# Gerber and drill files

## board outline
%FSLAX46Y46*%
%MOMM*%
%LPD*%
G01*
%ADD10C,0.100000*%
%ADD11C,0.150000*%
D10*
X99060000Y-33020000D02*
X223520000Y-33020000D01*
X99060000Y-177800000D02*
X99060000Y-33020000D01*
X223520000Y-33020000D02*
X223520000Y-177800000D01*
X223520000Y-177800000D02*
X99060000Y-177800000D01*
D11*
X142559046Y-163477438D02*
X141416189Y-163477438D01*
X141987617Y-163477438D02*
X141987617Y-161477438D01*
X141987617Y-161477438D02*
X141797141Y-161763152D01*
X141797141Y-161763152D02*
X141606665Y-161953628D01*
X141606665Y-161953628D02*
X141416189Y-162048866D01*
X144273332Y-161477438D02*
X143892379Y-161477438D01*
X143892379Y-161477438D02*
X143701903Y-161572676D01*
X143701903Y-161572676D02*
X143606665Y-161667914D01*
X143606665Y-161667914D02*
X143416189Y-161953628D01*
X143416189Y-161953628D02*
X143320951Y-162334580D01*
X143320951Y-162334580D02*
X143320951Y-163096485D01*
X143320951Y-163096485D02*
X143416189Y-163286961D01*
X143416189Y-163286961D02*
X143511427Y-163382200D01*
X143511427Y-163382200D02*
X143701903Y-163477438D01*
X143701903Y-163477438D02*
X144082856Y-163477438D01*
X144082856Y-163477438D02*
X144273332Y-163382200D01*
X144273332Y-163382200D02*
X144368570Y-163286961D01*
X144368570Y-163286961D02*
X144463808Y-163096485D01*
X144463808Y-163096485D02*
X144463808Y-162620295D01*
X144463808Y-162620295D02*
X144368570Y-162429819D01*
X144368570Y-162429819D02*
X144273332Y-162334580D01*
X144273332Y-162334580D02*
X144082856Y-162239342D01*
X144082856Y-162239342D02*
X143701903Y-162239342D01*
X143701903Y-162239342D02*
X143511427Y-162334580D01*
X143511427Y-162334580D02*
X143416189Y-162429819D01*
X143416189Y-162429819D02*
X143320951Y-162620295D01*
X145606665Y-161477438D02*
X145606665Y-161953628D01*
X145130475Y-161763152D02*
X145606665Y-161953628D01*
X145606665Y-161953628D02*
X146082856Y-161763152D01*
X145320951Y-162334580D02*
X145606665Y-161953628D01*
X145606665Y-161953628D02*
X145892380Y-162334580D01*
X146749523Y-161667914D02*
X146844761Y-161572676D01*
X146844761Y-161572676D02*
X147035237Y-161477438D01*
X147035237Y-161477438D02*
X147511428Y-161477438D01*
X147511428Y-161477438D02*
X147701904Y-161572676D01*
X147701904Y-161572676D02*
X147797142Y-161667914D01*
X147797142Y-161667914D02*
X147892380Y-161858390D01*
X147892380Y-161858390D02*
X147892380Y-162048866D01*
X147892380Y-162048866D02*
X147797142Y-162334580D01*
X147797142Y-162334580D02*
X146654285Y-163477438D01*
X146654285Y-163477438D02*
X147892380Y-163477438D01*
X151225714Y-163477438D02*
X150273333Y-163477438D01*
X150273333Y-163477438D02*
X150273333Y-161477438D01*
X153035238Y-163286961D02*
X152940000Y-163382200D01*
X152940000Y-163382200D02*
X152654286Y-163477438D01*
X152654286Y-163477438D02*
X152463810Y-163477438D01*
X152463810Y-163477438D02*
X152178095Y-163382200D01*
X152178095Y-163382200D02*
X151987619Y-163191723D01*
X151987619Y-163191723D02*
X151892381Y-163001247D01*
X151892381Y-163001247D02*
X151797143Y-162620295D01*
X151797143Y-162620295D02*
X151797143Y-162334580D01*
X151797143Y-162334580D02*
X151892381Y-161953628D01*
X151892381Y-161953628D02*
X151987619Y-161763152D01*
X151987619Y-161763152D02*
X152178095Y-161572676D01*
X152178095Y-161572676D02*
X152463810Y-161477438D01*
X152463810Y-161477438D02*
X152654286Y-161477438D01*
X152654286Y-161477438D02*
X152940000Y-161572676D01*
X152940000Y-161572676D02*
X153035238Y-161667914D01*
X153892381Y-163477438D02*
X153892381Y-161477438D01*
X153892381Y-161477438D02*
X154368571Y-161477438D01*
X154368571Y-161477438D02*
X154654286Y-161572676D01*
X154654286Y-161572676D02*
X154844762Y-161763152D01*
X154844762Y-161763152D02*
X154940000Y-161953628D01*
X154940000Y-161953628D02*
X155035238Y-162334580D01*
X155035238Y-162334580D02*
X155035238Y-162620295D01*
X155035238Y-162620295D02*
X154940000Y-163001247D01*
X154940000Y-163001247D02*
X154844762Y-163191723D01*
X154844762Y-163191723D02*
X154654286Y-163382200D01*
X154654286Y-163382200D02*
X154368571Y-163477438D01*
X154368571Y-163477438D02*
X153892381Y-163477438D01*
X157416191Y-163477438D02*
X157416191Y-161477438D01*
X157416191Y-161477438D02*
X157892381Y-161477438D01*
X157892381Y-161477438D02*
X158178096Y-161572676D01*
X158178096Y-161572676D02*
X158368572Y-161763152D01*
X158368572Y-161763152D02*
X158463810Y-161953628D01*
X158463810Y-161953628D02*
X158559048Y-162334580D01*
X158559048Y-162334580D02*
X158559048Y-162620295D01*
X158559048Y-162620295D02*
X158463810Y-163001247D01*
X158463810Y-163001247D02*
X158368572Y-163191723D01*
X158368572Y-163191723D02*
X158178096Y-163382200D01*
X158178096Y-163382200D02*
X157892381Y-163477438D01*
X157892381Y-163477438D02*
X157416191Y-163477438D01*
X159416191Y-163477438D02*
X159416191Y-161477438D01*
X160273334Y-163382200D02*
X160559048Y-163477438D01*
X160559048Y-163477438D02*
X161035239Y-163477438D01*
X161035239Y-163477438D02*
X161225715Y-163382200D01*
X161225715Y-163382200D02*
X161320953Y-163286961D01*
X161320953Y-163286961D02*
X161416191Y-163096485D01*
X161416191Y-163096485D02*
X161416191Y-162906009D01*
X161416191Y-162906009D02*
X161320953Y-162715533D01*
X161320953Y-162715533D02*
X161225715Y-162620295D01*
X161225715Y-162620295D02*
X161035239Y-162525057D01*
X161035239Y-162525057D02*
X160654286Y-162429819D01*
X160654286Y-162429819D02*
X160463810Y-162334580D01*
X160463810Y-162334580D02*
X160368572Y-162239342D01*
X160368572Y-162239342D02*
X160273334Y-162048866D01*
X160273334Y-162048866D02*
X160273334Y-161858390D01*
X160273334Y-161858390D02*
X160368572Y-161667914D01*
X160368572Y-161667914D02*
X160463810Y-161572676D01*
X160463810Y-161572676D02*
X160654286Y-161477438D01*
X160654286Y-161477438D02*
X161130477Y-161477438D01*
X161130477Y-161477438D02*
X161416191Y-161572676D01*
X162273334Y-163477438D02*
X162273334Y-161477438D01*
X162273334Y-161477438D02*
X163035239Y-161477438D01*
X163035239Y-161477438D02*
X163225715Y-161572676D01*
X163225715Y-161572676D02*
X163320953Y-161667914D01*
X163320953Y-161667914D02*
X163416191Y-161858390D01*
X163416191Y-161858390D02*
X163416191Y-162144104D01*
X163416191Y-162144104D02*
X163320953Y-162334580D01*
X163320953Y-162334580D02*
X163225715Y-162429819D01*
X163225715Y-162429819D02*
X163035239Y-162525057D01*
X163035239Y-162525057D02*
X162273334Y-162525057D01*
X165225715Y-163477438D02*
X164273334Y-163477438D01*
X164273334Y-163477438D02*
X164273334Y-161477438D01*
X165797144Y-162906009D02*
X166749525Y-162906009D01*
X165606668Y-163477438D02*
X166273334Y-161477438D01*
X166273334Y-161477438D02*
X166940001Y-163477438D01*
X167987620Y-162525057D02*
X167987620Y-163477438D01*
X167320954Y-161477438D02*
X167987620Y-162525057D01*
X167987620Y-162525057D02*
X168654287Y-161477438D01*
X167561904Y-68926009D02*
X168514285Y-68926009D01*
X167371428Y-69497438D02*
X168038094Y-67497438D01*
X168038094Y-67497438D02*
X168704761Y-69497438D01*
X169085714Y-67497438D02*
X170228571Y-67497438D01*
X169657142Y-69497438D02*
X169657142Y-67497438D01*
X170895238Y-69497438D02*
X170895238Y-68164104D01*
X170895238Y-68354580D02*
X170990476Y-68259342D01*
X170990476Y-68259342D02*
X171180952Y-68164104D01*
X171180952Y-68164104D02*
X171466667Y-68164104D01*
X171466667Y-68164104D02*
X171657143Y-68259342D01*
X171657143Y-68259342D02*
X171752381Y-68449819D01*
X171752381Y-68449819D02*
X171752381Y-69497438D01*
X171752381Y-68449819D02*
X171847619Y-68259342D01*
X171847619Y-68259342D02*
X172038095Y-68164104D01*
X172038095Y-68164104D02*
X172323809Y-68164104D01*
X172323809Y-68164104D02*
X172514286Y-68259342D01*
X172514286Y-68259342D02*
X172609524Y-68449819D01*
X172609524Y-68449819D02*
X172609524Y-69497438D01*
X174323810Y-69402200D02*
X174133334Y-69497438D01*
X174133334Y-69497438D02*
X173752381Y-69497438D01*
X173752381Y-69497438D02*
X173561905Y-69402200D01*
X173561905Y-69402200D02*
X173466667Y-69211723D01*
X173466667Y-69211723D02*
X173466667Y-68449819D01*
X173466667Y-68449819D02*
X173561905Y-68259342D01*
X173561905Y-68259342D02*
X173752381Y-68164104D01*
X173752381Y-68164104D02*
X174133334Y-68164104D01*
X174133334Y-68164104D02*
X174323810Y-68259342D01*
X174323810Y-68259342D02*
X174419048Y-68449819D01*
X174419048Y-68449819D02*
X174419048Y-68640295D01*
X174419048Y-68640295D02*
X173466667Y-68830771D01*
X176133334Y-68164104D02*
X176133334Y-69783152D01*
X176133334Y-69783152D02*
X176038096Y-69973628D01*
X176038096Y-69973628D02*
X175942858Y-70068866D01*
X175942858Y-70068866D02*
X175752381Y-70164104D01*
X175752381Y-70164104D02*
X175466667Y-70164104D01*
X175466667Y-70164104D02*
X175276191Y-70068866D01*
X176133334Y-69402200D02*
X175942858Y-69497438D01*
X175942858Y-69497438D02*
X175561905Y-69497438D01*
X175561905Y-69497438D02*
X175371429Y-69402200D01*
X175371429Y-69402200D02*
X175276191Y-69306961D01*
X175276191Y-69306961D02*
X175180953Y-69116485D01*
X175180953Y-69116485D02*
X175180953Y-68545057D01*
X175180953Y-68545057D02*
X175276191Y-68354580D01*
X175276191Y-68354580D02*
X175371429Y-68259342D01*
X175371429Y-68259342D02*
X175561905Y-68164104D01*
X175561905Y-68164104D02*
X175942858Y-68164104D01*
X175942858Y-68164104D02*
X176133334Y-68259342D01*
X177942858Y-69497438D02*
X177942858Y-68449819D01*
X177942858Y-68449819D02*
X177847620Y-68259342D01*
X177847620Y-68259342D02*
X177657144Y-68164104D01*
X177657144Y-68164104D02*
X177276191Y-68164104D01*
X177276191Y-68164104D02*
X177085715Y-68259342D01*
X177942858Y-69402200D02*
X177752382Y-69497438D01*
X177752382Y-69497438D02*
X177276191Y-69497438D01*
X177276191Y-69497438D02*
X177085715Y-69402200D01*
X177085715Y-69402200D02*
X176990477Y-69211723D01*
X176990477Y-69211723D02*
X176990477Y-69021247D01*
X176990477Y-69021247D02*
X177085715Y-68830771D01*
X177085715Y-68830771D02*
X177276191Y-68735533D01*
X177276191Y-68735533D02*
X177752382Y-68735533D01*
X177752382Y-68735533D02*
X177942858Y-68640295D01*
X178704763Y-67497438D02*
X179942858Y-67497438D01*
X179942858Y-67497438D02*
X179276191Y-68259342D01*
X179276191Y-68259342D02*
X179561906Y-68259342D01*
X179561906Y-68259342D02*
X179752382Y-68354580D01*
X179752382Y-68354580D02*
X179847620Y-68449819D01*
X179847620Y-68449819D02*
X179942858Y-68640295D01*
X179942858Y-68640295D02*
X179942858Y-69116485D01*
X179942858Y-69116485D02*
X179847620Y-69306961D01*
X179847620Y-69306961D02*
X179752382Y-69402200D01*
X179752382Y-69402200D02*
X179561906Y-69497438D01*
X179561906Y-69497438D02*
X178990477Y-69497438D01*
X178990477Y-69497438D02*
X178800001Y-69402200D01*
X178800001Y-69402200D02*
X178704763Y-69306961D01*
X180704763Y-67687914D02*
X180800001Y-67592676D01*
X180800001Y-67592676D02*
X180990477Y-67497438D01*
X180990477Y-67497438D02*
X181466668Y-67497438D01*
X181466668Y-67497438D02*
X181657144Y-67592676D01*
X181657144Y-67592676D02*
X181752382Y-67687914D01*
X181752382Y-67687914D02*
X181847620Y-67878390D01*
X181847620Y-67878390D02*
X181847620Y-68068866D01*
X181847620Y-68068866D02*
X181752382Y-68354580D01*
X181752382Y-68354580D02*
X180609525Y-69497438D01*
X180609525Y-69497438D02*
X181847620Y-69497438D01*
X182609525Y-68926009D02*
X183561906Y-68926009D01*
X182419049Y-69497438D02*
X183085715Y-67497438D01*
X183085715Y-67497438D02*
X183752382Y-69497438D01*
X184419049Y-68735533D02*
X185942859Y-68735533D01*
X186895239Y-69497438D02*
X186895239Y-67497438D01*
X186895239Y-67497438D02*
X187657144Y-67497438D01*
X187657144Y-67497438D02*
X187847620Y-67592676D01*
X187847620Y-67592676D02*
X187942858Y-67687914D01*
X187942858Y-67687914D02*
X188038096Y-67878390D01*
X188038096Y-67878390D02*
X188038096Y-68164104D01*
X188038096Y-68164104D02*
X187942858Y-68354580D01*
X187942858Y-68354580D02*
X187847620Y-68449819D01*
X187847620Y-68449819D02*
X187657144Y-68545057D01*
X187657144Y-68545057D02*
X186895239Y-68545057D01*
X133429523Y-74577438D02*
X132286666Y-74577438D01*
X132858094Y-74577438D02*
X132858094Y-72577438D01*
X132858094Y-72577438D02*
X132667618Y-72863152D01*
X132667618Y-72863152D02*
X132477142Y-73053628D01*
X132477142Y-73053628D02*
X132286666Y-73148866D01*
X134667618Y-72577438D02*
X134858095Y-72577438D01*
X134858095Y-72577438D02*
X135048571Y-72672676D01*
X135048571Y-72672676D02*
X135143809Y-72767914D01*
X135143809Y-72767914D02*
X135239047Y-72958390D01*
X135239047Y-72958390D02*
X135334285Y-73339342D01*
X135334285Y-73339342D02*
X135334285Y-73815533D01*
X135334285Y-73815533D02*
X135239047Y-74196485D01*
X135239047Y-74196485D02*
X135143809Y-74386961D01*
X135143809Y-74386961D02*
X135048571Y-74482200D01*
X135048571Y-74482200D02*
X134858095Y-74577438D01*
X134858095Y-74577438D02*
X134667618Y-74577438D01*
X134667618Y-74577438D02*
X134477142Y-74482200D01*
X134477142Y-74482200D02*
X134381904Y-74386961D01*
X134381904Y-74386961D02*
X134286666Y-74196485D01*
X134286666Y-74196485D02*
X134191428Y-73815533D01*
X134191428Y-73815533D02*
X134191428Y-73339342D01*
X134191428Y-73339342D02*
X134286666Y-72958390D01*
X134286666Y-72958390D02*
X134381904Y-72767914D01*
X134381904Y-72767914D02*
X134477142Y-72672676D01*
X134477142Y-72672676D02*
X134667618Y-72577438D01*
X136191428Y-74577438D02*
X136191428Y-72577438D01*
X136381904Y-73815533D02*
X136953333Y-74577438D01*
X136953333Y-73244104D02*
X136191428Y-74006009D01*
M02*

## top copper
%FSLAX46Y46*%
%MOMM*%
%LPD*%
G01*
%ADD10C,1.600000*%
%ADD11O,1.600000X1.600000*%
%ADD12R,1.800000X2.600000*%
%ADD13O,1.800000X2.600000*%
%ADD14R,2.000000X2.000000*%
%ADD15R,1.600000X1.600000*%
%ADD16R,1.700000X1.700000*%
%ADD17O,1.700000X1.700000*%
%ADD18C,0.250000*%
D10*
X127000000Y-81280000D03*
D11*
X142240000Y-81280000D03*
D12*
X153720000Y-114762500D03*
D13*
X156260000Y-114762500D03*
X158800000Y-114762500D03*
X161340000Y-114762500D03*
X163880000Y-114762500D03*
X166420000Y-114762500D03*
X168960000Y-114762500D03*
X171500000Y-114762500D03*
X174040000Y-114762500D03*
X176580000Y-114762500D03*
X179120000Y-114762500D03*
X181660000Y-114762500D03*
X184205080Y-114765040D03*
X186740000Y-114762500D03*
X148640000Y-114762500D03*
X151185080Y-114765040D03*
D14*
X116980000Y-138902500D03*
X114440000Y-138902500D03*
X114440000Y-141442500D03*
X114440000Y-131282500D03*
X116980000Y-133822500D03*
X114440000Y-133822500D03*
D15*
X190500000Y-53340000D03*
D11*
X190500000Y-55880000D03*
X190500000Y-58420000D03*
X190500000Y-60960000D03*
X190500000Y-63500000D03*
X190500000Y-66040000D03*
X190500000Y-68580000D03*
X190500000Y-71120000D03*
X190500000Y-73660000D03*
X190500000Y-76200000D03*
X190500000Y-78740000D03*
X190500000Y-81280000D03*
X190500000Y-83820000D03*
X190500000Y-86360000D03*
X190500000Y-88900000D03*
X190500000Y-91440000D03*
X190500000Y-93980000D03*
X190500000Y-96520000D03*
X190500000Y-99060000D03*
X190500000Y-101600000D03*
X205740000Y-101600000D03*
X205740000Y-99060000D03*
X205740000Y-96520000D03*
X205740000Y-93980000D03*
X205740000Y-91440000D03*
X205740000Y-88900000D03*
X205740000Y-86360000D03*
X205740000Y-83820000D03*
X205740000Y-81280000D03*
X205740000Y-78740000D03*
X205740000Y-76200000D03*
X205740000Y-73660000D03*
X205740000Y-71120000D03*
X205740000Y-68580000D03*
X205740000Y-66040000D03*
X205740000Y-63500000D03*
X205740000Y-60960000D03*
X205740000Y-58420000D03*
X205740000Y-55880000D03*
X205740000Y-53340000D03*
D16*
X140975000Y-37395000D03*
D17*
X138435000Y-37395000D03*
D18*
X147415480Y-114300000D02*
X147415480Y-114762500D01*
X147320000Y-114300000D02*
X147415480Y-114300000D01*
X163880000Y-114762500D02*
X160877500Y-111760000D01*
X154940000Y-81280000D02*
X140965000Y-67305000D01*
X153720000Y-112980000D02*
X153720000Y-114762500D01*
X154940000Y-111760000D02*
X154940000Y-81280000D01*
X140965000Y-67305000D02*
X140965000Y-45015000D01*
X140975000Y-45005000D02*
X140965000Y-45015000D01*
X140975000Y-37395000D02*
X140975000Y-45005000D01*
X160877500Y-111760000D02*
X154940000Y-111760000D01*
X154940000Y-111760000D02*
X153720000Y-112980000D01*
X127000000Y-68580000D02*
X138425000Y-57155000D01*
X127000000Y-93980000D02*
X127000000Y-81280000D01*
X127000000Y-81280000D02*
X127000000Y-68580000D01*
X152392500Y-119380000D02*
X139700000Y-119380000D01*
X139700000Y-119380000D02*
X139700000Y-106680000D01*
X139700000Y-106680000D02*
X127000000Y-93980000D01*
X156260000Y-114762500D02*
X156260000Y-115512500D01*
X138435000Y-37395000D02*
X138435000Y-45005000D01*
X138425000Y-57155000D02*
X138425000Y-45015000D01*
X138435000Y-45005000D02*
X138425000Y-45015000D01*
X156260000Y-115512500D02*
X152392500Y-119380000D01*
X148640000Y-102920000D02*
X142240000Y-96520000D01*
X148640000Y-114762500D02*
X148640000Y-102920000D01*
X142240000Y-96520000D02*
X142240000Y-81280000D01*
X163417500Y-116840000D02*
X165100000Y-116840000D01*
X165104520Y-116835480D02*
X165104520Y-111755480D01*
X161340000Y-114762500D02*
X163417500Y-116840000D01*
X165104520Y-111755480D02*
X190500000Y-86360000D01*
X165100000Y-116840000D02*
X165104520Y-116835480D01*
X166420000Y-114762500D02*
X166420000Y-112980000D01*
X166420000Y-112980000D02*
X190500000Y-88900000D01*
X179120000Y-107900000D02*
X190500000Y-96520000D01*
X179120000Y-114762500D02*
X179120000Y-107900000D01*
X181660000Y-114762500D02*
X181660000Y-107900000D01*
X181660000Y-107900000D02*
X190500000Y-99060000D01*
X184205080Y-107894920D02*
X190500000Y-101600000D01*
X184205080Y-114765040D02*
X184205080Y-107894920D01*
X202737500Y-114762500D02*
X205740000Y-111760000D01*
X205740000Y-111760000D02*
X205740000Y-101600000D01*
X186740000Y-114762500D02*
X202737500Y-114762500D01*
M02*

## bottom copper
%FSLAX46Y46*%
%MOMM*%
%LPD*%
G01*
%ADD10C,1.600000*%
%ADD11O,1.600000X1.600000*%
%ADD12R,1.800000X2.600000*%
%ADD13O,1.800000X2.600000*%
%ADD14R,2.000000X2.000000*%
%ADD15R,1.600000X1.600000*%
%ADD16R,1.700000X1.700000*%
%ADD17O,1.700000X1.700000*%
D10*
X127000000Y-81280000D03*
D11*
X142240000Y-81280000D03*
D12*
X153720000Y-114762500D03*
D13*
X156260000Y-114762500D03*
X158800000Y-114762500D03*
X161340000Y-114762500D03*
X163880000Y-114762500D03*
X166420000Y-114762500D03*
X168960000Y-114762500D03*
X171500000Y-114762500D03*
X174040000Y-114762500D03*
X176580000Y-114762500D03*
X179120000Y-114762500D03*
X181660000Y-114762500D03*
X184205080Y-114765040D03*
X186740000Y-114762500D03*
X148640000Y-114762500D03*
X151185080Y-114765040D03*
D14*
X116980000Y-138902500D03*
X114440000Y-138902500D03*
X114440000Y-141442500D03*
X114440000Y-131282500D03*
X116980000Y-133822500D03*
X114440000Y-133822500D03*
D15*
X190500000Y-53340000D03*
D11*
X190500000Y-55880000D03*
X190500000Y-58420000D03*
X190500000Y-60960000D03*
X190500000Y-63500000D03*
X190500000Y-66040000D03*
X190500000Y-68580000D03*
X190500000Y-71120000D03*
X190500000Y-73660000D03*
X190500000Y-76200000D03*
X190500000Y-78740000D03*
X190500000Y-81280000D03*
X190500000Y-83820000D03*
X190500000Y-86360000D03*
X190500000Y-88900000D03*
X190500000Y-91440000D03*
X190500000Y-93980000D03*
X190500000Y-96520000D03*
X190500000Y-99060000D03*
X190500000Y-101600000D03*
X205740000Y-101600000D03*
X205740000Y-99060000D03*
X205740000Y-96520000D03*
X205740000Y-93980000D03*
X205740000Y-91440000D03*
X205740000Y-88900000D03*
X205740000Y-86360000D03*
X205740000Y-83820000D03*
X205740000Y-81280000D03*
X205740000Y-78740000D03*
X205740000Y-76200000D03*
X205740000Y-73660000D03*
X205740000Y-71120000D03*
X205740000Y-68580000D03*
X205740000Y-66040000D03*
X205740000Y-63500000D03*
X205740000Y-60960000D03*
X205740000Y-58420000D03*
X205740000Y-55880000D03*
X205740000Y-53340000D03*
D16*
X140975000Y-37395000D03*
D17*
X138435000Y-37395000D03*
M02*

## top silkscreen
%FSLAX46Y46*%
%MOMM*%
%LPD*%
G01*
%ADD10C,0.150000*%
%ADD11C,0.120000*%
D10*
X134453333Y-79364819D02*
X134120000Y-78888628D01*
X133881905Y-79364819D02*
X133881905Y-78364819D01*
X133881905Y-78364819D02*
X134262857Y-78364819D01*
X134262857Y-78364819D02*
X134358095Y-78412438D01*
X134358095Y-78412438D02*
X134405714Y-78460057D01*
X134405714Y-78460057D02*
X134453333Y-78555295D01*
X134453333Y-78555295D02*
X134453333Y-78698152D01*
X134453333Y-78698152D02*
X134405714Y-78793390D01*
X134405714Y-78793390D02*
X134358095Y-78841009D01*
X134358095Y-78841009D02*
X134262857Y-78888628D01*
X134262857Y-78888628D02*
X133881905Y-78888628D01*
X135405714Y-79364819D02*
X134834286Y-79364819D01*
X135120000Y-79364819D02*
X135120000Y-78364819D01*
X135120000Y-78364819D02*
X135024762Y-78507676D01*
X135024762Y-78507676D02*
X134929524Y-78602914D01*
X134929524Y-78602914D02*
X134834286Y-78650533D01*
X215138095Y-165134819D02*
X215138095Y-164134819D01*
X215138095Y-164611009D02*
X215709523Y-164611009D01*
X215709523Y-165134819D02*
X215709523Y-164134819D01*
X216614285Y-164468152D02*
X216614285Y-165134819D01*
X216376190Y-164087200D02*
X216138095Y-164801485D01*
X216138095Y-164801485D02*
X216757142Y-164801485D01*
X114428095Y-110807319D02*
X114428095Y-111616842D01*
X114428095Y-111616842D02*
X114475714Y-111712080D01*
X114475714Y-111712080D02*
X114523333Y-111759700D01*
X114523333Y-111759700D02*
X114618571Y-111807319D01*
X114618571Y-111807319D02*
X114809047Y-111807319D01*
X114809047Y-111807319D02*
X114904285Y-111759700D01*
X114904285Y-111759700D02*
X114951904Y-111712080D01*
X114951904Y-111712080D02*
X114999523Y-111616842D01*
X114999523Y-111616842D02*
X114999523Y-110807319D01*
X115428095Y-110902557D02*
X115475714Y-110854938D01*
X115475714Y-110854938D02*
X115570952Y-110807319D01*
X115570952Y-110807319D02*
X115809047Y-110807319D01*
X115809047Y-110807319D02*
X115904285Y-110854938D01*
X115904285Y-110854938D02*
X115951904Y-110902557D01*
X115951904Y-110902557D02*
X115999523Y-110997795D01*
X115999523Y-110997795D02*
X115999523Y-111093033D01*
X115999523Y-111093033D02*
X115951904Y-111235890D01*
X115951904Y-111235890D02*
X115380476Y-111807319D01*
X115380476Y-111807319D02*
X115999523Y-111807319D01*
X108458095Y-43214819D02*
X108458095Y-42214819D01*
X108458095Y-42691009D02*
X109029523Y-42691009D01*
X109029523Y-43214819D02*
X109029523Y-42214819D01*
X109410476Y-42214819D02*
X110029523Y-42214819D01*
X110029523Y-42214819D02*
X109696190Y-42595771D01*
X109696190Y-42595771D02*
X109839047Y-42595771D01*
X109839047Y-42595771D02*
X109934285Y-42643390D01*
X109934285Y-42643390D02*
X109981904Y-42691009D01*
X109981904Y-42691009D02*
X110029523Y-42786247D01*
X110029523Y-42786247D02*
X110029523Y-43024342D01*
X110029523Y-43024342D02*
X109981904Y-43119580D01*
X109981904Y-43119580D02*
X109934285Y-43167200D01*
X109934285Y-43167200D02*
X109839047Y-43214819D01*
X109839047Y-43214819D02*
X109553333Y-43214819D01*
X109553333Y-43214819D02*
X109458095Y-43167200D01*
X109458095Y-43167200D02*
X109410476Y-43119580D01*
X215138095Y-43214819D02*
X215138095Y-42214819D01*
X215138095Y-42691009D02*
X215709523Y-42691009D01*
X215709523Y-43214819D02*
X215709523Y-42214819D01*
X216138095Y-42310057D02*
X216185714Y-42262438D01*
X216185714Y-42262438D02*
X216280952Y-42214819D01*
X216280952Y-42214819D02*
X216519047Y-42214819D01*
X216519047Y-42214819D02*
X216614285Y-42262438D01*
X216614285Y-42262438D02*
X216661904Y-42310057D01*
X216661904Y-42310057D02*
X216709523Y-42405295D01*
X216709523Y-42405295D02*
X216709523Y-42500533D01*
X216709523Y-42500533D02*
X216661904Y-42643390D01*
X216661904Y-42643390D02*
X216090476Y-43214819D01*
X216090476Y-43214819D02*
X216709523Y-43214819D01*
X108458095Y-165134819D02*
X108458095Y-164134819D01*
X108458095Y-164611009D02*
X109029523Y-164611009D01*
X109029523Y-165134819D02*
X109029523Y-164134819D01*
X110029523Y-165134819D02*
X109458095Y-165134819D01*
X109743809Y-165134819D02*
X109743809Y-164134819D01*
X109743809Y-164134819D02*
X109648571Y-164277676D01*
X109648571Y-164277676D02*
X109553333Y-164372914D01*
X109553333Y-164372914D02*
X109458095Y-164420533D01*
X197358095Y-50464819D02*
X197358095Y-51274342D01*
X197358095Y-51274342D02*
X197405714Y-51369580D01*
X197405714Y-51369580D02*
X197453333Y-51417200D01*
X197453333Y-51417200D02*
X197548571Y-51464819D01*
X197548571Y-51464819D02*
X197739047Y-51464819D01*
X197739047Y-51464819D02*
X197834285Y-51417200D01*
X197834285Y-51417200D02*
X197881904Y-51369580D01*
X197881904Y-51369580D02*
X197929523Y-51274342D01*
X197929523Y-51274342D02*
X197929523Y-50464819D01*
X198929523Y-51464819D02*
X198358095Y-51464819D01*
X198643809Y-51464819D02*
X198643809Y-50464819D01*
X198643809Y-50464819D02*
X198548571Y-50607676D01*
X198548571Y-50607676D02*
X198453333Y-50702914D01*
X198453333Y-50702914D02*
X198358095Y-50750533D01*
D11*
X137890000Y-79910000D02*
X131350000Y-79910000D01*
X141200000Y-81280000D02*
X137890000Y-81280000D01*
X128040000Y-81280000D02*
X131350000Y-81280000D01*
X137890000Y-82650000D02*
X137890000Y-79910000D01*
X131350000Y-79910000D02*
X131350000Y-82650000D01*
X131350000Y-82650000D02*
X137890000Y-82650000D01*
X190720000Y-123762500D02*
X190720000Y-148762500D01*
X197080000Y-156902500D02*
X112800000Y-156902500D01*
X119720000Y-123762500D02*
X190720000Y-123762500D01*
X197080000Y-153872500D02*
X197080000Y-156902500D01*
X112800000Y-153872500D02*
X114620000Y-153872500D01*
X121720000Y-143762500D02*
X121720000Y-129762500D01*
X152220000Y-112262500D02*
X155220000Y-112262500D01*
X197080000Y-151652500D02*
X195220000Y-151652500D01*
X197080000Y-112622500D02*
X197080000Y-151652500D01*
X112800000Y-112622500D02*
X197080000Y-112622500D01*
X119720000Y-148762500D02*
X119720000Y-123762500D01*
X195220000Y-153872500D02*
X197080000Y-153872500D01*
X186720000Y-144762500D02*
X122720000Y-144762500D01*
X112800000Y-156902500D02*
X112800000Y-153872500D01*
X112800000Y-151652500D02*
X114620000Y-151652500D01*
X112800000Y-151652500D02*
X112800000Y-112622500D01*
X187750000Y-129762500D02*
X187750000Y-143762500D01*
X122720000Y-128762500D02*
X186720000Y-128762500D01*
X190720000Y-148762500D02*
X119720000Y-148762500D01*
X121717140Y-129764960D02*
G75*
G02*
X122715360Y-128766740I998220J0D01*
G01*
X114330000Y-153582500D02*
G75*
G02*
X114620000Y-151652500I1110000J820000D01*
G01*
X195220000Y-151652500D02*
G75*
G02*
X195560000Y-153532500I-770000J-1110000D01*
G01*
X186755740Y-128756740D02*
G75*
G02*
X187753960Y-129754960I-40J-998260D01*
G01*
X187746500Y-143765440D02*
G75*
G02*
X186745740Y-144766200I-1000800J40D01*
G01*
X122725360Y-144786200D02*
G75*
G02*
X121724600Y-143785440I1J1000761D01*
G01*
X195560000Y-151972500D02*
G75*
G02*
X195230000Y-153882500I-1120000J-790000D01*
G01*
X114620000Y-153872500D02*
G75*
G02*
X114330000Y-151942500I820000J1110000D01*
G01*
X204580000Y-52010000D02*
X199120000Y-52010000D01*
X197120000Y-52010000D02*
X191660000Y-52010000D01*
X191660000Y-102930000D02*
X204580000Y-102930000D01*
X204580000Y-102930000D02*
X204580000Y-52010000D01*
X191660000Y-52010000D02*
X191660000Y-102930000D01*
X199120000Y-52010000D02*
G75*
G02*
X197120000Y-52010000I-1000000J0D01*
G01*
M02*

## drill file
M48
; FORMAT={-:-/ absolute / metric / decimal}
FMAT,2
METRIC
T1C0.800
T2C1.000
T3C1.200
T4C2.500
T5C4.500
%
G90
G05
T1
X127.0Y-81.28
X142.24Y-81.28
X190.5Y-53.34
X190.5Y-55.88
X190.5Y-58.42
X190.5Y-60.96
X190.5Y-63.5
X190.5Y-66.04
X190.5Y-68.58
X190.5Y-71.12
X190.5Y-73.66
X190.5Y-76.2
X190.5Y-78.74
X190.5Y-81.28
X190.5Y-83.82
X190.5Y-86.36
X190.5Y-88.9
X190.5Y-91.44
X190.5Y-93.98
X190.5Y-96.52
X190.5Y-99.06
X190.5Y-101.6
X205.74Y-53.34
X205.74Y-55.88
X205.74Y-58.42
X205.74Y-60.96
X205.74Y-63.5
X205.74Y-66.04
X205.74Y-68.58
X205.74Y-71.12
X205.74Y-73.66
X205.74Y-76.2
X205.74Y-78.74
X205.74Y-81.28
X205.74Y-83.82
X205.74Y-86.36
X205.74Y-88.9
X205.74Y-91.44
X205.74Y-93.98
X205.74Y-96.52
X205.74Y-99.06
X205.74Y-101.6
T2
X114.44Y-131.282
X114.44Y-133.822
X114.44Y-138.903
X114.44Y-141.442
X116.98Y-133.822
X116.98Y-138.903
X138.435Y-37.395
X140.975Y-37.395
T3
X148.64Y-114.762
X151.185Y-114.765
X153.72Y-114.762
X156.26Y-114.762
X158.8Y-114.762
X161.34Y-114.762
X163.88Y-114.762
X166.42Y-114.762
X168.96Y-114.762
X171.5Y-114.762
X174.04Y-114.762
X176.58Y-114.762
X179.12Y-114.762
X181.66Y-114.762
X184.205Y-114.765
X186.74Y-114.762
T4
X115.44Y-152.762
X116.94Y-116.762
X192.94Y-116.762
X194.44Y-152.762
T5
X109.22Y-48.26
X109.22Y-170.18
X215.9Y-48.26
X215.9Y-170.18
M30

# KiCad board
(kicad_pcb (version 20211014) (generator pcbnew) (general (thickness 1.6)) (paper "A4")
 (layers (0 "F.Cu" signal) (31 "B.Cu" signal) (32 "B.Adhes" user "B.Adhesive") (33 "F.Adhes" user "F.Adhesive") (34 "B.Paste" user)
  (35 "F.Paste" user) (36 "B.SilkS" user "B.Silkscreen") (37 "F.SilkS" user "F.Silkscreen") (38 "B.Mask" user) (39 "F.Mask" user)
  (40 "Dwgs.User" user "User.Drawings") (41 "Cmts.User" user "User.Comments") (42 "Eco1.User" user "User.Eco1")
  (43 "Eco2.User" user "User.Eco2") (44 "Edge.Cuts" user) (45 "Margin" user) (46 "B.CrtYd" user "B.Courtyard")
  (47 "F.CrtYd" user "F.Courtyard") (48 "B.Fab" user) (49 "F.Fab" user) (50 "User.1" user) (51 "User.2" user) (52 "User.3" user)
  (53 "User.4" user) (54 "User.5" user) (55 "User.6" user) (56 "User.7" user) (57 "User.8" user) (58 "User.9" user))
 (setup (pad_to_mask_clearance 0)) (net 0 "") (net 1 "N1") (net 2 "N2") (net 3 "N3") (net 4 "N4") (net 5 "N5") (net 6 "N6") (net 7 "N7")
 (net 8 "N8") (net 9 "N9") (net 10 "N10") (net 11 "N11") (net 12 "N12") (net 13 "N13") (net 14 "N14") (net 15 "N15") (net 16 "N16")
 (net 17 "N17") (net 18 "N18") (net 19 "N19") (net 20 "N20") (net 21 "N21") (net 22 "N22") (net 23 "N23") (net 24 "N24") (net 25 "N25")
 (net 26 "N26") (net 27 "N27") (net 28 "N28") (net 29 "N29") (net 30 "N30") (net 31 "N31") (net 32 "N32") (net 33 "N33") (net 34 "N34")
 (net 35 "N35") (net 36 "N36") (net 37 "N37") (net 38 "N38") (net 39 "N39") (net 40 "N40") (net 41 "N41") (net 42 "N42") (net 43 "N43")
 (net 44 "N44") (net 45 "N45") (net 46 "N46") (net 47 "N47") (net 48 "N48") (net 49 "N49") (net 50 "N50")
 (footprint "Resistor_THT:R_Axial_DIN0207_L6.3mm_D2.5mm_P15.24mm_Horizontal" (layer "F.Cu") (at 127 81.28)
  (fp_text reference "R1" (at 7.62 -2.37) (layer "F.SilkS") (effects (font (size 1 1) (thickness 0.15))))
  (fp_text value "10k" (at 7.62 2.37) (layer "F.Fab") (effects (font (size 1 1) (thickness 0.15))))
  (fp_line (start 10.89 -1.37) (end 4.35 -1.37) (layer "F.SilkS") (width 0.12))
  (fp_line (start 14.2 0) (end 10.89 0) (layer "F.SilkS") (width 0.12))
  (fp_line (start 1.04 0) (end 4.35 0) (layer "F.SilkS") (width 0.12))
  (fp_line (start 10.89 1.37) (end 10.89 -1.37) (layer "F.SilkS") (width 0.12))
  (fp_line (start 4.35 -1.37) (end 4.35 1.37) (layer "F.SilkS") (width 0.12))
  (fp_line (start 4.35 1.37) (end 10.89 1.37) (layer "F.SilkS") (width 0.12))
  (pad "1" thru_hole circle (at 0 0) (size 1.6 1.6) (drill 0.8) (layers *.Cu *.Mask) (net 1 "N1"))
  (pad "2" thru_hole oval (at 15.24 0) (size 1.6 1.6) (drill 0.8) (layers *.Cu *.Mask) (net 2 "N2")))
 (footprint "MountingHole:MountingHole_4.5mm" (layer "F.Cu") (at 215.9 170.18)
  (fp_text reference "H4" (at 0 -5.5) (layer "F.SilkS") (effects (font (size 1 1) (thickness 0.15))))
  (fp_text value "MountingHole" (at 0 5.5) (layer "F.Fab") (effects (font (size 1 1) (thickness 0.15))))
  (pad "" np_thru_hole circle (at 0 0) (size 4.5 4.5) (drill 4.5) (layers *.Cu *.Mask)))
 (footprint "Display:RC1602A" (layer "F.Cu") (at 153.72 114.7625)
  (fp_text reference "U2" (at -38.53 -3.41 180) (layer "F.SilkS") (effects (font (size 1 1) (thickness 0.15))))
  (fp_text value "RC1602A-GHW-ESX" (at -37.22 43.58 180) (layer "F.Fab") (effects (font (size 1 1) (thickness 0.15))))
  (fp_line (start 37 9) (end 37 34) (layer "F.SilkS") (width 0.12))
  (fp_line (start 43.36 42.14) (end -40.92 42.14) (layer "F.SilkS") (width 0.12))
  (fp_line (start -34 9) (end 37 9) (layer "F.SilkS") (width 0.12))
  (fp_line (start 43.36 39.11) (end 43.36 42.14) (layer "F.SilkS") (width 0.12))
  (fp_line (start -40.92 39.11) (end -39.1 39.11) (layer "F.SilkS") (width 0.12))
  (fp_line (start -32 29) (end -32 15) (layer "F.SilkS") (width 0.12))
  (fp_line (start -1.5 -2.5) (end 1.5 -2.5) (layer "F.SilkS") (width 0.12))
  (fp_line (start 43.36 36.89) (end 41.5 36.89) (layer "F.SilkS") (width 0.12))
  (fp_line (start 43.36 -2.14) (end 43.36 36.89) (layer "F.SilkS") (width 0.12))
  (fp_line (start -40.92 -2.14) (end 43.36 -2.14) (layer "F.SilkS") (width 0.12))
  (fp_line (start -34 34) (end -34 9) (layer "F.SilkS") (width 0.12))
  (fp_line (start 41.5 39.11) (end 43.36 39.11) (layer "F.SilkS") (width 0.12))
  (fp_line (start 33 30) (end -31 30) (layer "F.SilkS") (width 0.12))
  (fp_line (start -40.92 42.14) (end -40.92 39.11) (layer "F.SilkS") (width 0.12))
  (fp_line (start -40.92 36.89) (end -39.1 36.89) (layer "F.SilkS") (width 0.12))
  (fp_line (start -40.92 36.89) (end -40.92 -2.14) (layer "F.SilkS") (width 0.12))
  (fp_line (start 34.03 15) (end 34.03 29) (layer "F.SilkS") (width 0.12))
  (fp_line (start -31 14) (end 33 14) (layer "F.SilkS") (width 0.12))
  (fp_line (start 37 34) (end -34 34) (layer "F.SilkS") (width 0.12))
  (fp_arc (start -32.00286 15.00246) (mid -31.710488 14.296612) (end -31.00464 14.00424) (layer "F.SilkS") (width 0.12))
  (fp_arc (start -39.39 38.82) (mid -39.644716 37.794939) (end -39.1 36.89) (layer "F.SilkS") (width 0.12))
  (fp_arc (start 41.5 36.89) (mid 42.059361 37.759584) (end 41.84 38.77) (layer "F.SilkS") (width 0.12))
  (fp_arc (start 33.03574 13.99424) (mid 33.741576 14.286624) (end 34.03396 14.99246) (layer "F.SilkS") (width 0.12))
  (fp_arc (start 34.0265 29.00294) (mid 33.733372 29.710572) (end 33.02574 30.0037) (layer "F.SilkS") (width 0.12))
  (fp_arc (start -30.99464 30.0237) (mid -31.702284 29.730584) (end -31.9954 29.02294) (layer "F.SilkS") (width 0.12))
  (fp_arc (start 41.84 37.21) (mid 42.070574 38.233345) (end 41.51 39.12) (layer "F.SilkS") (width 0.12))
  (fp_arc (start -39.1 39.11) (mid -39.644716 38.205061) (end -39.39 37.18) (layer "F.SilkS") (width 0.12))
  (pad "" np_thru_hole circle (at 40.72 38 180) (size 2.5 2.5) (drill 2.5) (layers *.Cu *.Mask))
  (pad "" np_thru_hole circle (at 39.22 2 180) (size 2.5 2.5) (drill 2.5) (layers *.Cu *.Mask))
  (pad "" np_thru_hole circle (at -38.28 38 180) (size 2.5 2.5) (drill 2.5) (layers *.Cu *.Mask))
  (pad "" np_thru_hole circle (at -36.78 2 180) (size 2.5 2.5) (drill 2.5) (layers *.Cu *.Mask))
  (pad "1" thru_hole rect (at 0 0 180) (size 1.8 2.6) (drill 1.2) (layers *.Cu *.Mask) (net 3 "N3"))
  (pad "2" thru_hole oval (at 2.54 0 180) (size 1.8 2.6) (drill 1.2) (layers *.Cu *.Mask) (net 1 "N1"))
  (pad "3" thru_hole oval (at 5.08 0 180) (size 1.8 2.6) (drill 1.2) (layers *.Cu *.Mask) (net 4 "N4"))
  (pad "4" thru_hole oval (at 7.62 0 180) (size 1.8 2.6) (drill 1.2) (layers *.Cu *.Mask) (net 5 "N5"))
  (pad "5" thru_hole oval (at 10.16 0 180) (size 1.8 2.6) (drill 1.2) (layers *.Cu *.Mask) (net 3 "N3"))
  (pad "6" thru_hole oval (at 12.7 0 180) (size 1.8 2.6) (drill 1.2) (layers *.Cu *.Mask) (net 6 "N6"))
  (pad "7" thru_hole oval (at 15.24 0 180) (size 1.8 2.6) (drill 1.2) (layers *.Cu *.Mask) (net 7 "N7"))
  (pad "8" thru_hole oval (at 17.78 0 180) (size 1.8 2.6) (drill 1.2) (layers *.Cu *.Mask) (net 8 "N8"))
  (pad "9" thru_hole oval (at 20.32 0 180) (size 1.8 2.6) (drill 1.2) (layers *.Cu *.Mask) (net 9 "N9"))
  (pad "10" thru_hole oval (at 22.86 0 180) (size 1.8 2.6) (drill 1.2) (layers *.Cu *.Mask) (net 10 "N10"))
  (pad "11" thru_hole oval (at 25.4 0 180) (size 1.8 2.6) (drill 1.2) (layers *.Cu *.Mask) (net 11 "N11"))
  (pad "12" thru_hole oval (at 27.94 0 180) (size 1.8 2.6) (drill 1.2) (layers *.Cu *.Mask) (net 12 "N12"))
  (pad "13" thru_hole oval (at 30.48508 0.00254 180) (size 1.8 2.6) (drill 1.2) (layers *.Cu *.Mask) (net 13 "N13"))
  (pad "14" thru_hole oval (at 33.02 0 180) (size 1.8 2.6) (drill 1.2) (layers *.Cu *.Mask) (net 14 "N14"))
  (pad "15" thru_hole oval (at -5.08 0 180) (size 1.8 2.6) (drill 1.2) (layers *.Cu *.Mask) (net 2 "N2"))
  (pad "16" thru_hole oval (at -2.53492 0.00254 180) (size 1.8 2.6) (drill 1.2) (layers *.Cu *.Mask) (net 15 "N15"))
  (pad "A1" thru_hole rect (at -36.74 24.14 180) (size 2 2) (drill 1) (layers *.Cu *.Mask) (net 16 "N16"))
  (pad "A1" thru_hole rect (at -39.28 24.14 180) (size 2 2) (drill 1) (layers *.Cu *.Mask) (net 16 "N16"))
  (pad "A1" thru_hole rect (at -39.28 26.68 180) (size 2 2) (drill 1) (layers *.Cu *.Mask) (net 16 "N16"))
  (pad "K1" thru_hole rect (at -39.28 16.52 180) (size 2 2) (drill 1) (layers *.Cu *.Mask) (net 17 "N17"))
  (pad "K1" thru_hole rect (at -36.74 19.06 180) (size 2 2) (drill 1) (layers *.Cu *.Mask) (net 17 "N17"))
  (pad "K1" thru_hole rect (at -39.28 19.06 180) (size 2 2) (drill 1) (layers *.Cu *.Mask) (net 17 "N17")))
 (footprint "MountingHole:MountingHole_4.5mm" (layer "F.Cu") (at 109.22 48.26)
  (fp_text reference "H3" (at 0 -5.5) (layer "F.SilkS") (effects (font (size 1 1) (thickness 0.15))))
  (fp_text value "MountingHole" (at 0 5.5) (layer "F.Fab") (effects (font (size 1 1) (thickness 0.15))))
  (pad "" np_thru_hole circle (at 0 0) (size 4.5 4.5) (drill 4.5) (layers *.Cu *.Mask)))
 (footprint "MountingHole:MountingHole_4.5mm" (layer "F.Cu") (at 215.9 48.26)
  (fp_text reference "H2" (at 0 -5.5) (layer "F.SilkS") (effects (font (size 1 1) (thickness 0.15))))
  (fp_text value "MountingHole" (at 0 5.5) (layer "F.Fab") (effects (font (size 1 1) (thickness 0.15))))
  (pad "" np_thru_hole circle (at 0 0) (size 4.5 4.5) (drill 4.5) (layers *.Cu *.Mask)))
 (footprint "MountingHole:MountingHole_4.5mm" (layer "F.Cu") (at 109.22 170.18)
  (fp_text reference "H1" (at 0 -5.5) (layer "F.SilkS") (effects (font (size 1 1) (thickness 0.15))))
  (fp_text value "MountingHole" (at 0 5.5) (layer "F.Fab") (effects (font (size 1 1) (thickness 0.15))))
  (pad "" np_thru_hole circle (at 0 0) (size 4.5 4.5) (drill 4.5) (layers *.Cu *.Mask)))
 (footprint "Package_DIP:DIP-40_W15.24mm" (layer "F.Cu") (at 190.5 53.34)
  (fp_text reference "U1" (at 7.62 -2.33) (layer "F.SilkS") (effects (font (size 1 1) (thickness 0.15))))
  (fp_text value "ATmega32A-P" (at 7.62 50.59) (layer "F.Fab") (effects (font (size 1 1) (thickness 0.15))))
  (fp_line (start 14.08 -1.33) (end 8.62 -1.33) (layer "F.SilkS") (width 0.12))
  (fp_line (start 6.62 -1.33) (end 1.16 -1.33) (layer "F.SilkS") (width 0.12))
  (fp_line (start 1.16 49.59) (end 14.08 49.59) (layer "F.SilkS") (width 0.12))
  (fp_line (start 14.08 49.59) (end 14.08 -1.33) (layer "F.SilkS") (width 0.12))
  (fp_line (start 1.16 -1.33) (end 1.16 49.59) (layer "F.SilkS") (width 0.12))
  (fp_arc (start 8.62 -1.33) (mid 7.62 -0.33) (end 6.62 -1.33) (layer "F.SilkS") (width 0.12))
  (pad "1" thru_hole rect (at 0 0) (size 1.6 1.6) (drill 0.8) (layers *.Cu *.Mask) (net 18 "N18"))
  (pad "2" thru_hole oval (at 0 2.54) (size 1.6 1.6) (drill 0.8) (layers *.Cu *.Mask) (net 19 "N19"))
  (pad "3" thru_hole oval (at 0 5.08) (size 1.6 1.6) (drill 0.8) (layers *.Cu *.Mask) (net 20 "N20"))
  (pad "4" thru_hole oval (at 0 7.62) (size 1.6 1.6) (drill 0.8) (layers *.Cu *.Mask) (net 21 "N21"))
  (pad "5" thru_hole oval (at 0 10.16) (size 1.6 1.6) (drill 0.8) (layers *.Cu *.Mask) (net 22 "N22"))
  (pad "6" thru_hole oval (at 0 12.7) (size 1.6 1.6) (drill 0.8) (layers *.Cu *.Mask) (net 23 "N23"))
  (pad "7" thru_hole oval (at 0 15.24) (size 1.6 1.6) (drill 0.8) (layers *.Cu *.Mask) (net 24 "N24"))
  (pad "8" thru_hole oval (at 0 17.78) (size 1.6 1.6) (drill 0.8) (layers *.Cu *.Mask) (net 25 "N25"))
  (pad "9" thru_hole oval (at 0 20.32) (size 1.6 1.6) (drill 0.8) (layers *.Cu *.Mask) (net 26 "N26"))
  (pad "10" thru_hole oval (at 0 22.86) (size 1.6 1.6) (drill 0.8) (layers *.Cu *.Mask) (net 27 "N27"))
  (pad "11" thru_hole oval (at 0 25.4) (size 1.6 1.6) (drill 0.8) (layers *.Cu *.Mask) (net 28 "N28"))
  (pad "12" thru_hole oval (at 0 27.94) (size 1.6 1.6) (drill 0.8) (layers *.Cu *.Mask) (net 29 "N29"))
  (pad "13" thru_hole oval (at 0 30.48) (size 1.6 1.6) (drill 0.8) (layers *.Cu *.Mask) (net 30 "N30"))
  (pad "14" thru_hole oval (at 0 33.02) (size 1.6 1.6) (drill 0.8) (layers *.Cu *.Mask) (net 5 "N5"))
  (pad "15" thru_hole oval (at 0 35.56) (size 1.6 1.6) (drill 0.8) (layers *.Cu *.Mask) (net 6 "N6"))
  (pad "16" thru_hole oval (at 0 38.1) (size 1.6 1.6) (drill 0.8) (layers *.Cu *.Mask) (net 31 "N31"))
  (pad "17" thru_hole oval (at 0 40.64) (size 1.6 1.6) (drill 0.8) (layers *.Cu *.Mask) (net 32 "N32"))
  (pad "18" thru_hole oval (at 0 43.18) (size 1.6 1.6) (drill 0.8) (layers *.Cu *.Mask) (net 11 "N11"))
  (pad "19" thru_hole oval (at 0 45.72) (size 1.6 1.6) (drill 0.8) (layers *.Cu *.Mask) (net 12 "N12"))
  (pad "20" thru_hole oval (at 0 48.26) (size 1.6 1.6) (drill 0.8) (layers *.Cu *.Mask) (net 13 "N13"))
  (pad "21" thru_hole oval (at 15.24 48.26) (size 1.6 1.6) (drill 0.8) (layers *.Cu *.Mask) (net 14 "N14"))
  (pad "22" thru_hole oval (at 15.24 45.72) (size 1.6 1.6) (drill 0.8) (layers *.Cu *.Mask) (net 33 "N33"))
  (pad "23" thru_hole oval (at 15.24 43.18) (size 1.6 1.6) (drill 0.8) (layers *.Cu *.Mask) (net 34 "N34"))
  (pad "24" thru_hole oval (at 15.24 40.64) (size 1.6 1.6) (drill 0.8) (layers *.Cu *.Mask) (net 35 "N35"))
  (pad "25" thru_hole oval (at 15.24 38.1) (size 1.6 1.6) (drill 0.8) (layers *.Cu *.Mask) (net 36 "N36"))
  (pad "26" thru_hole oval (at 15.24 35.56) (size 1.6 1.6) (drill 0.8) (layers *.Cu *.Mask) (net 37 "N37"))
  (pad "27" thru_hole oval (at 15.24 33.02) (size 1.6 1.6) (drill 0.8) (layers *.Cu *.Mask) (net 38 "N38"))
  (pad "28" thru_hole oval (at 15.24 30.48) (size 1.6 1.6) (drill 0.8) (layers *.Cu *.Mask) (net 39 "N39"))
  (pad "29" thru_hole oval (at 15.24 27.94) (size 1.6 1.6) (drill 0.8) (layers *.Cu *.Mask) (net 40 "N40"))
  (pad "30" thru_hole oval (at 15.24 25.4) (size 1.6 1.6) (drill 0.8) (layers *.Cu *.Mask) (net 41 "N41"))
  (pad "31" thru_hole oval (at 15.24 22.86) (size 1.6 1.6) (drill 0.8) (layers *.Cu *.Mask) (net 28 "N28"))
  (pad "32" thru_hole oval (at 15.24 20.32) (size 1.6 1.6) (drill 0.8) (layers *.Cu *.Mask) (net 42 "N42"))
  (pad "33" thru_hole oval (at 15.24 17.78) (size 1.6 1.6) (drill 0.8) (layers *.Cu *.Mask) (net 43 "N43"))
  (pad "34" thru_hole oval (at 15.24 15.24) (size 1.6 1.6) (drill 0.8) (layers *.Cu *.Mask) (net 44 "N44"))
  (pad "35" thru_hole oval (at 15.24 12.7) (size 1.6 1.6) (drill 0.8) (layers *.Cu *.Mask) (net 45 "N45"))
  (pad "36" thru_hole oval (at 15.24 10.16) (size 1.6 1.6) (drill 0.8) (layers *.Cu *.Mask) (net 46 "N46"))
  (pad "37" thru_hole oval (at 15.24 7.62) (size 1.6 1.6) (drill 0.8) (layers *.Cu *.Mask) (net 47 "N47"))
  (pad "38" thru_hole oval (at 15.24 5.08) (size 1.6 1.6) (drill 0.8) (layers *.Cu *.Mask) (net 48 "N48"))
  (pad "39" thru_hole oval (at 15.24 2.54) (size 1.6 1.6) (drill 0.8) (layers *.Cu *.Mask) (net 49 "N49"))
  (pad "40" thru_hole oval (at 15.24 0) (size 1.6 1.6) (drill 0.8) (layers *.Cu *.Mask) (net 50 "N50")))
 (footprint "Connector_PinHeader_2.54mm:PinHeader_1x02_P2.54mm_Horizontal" (layer "B.Cu") (at 140.975 37.395 90)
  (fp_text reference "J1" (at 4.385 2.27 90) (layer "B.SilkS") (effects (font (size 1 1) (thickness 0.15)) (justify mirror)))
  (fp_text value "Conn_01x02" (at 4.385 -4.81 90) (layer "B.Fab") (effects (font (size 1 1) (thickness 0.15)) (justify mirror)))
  (pad "1" thru_hole rect (at 0 0 90) (size 1.7 1.7) (drill 1) (layers *.Cu *.Mask) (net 3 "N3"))
  (pad "2" thru_hole oval (at 0 -2.54 90) (size 1.7 1.7) (drill 1) (layers *.Cu *.Mask) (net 1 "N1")))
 (gr_line (start 99.06 33.02) (end 223.52 33.02) (layer "Edge.Cuts") (width 0.1))
 (gr_line (start 99.06 177.8) (end 99.06 33.02) (layer "Edge.Cuts") (width 0.1))
 (gr_line (start 223.52 33.02) (end 223.52 177.8) (layer "Edge.Cuts") (width 0.1))
 (gr_line (start 223.52 177.8) (end 99.06 177.8) (layer "Edge.Cuts") (width 0.1))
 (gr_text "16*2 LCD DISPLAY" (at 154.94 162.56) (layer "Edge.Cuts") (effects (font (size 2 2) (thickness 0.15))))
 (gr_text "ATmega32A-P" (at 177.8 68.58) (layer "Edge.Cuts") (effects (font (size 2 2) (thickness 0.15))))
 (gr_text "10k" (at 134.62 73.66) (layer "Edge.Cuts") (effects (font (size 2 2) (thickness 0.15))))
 (segment (start 147.41548 114.3) (end 147.41548 114.7625) (width 0.25) (layer "F.Cu") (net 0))
 (segment (start 147.32 114.3) (end 147.41548 114.3) (width 0.25) (layer "F.Cu") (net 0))
 (segment (start 163.88 114.7625) (end 160.8775 111.76) (width 0.25) (layer "F.Cu") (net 3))
 (segment (start 154.94 81.28) (end 140.965 67.305) (width 0.25) (layer "F.Cu") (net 3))
 (segment (start 153.72 112.98) (end 153.72 114.7625) (width 0.25) (layer "F.Cu") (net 3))
 (segment (start 154.94 111.76) (end 154.94 81.28) (width 0.25) (layer "F.Cu") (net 3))
 (segment (start 140.965 67.305) (end 140.965 45.015) (width 0.25) (layer "F.Cu") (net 3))
 (segment (start 140.975 45.005) (end 140.965 45.015) (width 0.25) (layer "F.Cu") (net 3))
 (segment (start 140.975 37.395) (end 140.975 45.005) (width 0.25) (layer "F.Cu") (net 3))
 (segment (start 160.8775 111.76) (end 154.94 111.76) (width 0.25) (layer "F.Cu") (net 3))
 (segment (start 154.94 111.76) (end 153.72 112.98) (width 0.25) (layer "F.Cu") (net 3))
 (segment (start 127 68.58) (end 138.425 57.155) (width 0.25) (layer "F.Cu") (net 1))
 (segment (start 127 93.98) (end 127 81.28) (width 0.25) (layer "F.Cu") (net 1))
 (segment (start 127 81.28) (end 127 68.58) (width 0.25) (layer "F.Cu") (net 1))
 (segment (start 152.3925 119.38) (end 139.7 119.38) (width 0.25) (layer "F.Cu") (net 1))
 (segment (start 139.7 119.38) (end 139.7 106.68) (width 0.25) (layer "F.Cu") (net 1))
 (segment (start 139.7 106.68) (end 127 93.98) (width 0.25) (layer "F.Cu") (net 1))
 (segment (start 156.26 114.7625) (end 156.26 115.5125) (width 0.25) (layer "F.Cu") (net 1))
 (segment (start 138.435 37.395) (end 138.435 45.005) (width 0.25) (layer "F.Cu") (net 1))
 (segment (start 138.425 57.155) (end 138.425 45.015) (width 0.25) (layer "F.Cu") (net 1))
 (segment (start 138.435 45.005) (end 138.425 45.015) (width 0.25) (layer "F.Cu") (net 1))
 (segment (start 156.26 115.5125) (end 152.3925 119.38) (width 0.25) (layer "F.Cu") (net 1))
 (segment (start 148.64 102.92) (end 142.24 96.52) (width 0.25) (layer "F.Cu") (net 2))
 (segment (start 148.64 114.7625) (end 148.64 102.92) (width 0.25) (layer "F.Cu") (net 2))
 (segment (start 142.24 96.52) (end 142.24 81.28) (width 0.25) (layer "F.Cu") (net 2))
 (segment (start 163.4175 116.84) (end 165.1 116.84) (width 0.25) (layer "F.Cu") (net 5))
 (segment (start 165.10452 116.83548) (end 165.10452 111.75548) (width 0.25) (layer "F.Cu") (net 5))
 (segment (start 161.34 114.7625) (end 163.4175 116.84) (width 0.25) (layer "F.Cu") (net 5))
 (segment (start 165.10452 111.75548) (end 190.5 86.36) (width 0.25) (layer "F.Cu") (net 5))
 (segment (start 165.1 116.84) (end 165.10452 116.83548) (width 0.25) (layer "F.Cu") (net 5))
 (segment (start 166.42 114.7625) (end 166.42 112.98) (width 0.25) (layer "F.Cu") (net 6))
 (segment (start 166.42 112.98) (end 190.5 88.9) (width 0.25) (layer "F.Cu") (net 6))
 (segment (start 179.12 107.9) (end 190.5 96.52) (width 0.25) (layer "F.Cu") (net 11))
 (segment (start 179.12 114.7625) (end 179.12 107.9) (width 0.25) (layer "F.Cu") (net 11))
 (segment (start 181.66 114.7625) (end 181.66 107.9) (width 0.25) (layer "F.Cu") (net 12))
 (segment (start 181.66 107.9) (end 190.5 99.06) (width 0.25) (layer "F.Cu") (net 12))
 (segment (start 184.20508 107.89492) (end 190.5 101.6) (width 0.25) (layer "F.Cu") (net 13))
 (segment (start 184.20508 114.76504) (end 184.20508 107.89492) (width 0.25) (layer "F.Cu") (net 13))
 (segment (start 202.7375 114.7625) (end 205.74 111.76) (width 0.25) (layer "F.Cu") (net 14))
 (segment (start 205.74 111.76) (end 205.74 101.6) (width 0.25) (layer "F.Cu") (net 14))
 (segment (start 186.74 114.7625) (end 202.7375 114.7625) (width 0.25) (layer "F.Cu") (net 14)))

